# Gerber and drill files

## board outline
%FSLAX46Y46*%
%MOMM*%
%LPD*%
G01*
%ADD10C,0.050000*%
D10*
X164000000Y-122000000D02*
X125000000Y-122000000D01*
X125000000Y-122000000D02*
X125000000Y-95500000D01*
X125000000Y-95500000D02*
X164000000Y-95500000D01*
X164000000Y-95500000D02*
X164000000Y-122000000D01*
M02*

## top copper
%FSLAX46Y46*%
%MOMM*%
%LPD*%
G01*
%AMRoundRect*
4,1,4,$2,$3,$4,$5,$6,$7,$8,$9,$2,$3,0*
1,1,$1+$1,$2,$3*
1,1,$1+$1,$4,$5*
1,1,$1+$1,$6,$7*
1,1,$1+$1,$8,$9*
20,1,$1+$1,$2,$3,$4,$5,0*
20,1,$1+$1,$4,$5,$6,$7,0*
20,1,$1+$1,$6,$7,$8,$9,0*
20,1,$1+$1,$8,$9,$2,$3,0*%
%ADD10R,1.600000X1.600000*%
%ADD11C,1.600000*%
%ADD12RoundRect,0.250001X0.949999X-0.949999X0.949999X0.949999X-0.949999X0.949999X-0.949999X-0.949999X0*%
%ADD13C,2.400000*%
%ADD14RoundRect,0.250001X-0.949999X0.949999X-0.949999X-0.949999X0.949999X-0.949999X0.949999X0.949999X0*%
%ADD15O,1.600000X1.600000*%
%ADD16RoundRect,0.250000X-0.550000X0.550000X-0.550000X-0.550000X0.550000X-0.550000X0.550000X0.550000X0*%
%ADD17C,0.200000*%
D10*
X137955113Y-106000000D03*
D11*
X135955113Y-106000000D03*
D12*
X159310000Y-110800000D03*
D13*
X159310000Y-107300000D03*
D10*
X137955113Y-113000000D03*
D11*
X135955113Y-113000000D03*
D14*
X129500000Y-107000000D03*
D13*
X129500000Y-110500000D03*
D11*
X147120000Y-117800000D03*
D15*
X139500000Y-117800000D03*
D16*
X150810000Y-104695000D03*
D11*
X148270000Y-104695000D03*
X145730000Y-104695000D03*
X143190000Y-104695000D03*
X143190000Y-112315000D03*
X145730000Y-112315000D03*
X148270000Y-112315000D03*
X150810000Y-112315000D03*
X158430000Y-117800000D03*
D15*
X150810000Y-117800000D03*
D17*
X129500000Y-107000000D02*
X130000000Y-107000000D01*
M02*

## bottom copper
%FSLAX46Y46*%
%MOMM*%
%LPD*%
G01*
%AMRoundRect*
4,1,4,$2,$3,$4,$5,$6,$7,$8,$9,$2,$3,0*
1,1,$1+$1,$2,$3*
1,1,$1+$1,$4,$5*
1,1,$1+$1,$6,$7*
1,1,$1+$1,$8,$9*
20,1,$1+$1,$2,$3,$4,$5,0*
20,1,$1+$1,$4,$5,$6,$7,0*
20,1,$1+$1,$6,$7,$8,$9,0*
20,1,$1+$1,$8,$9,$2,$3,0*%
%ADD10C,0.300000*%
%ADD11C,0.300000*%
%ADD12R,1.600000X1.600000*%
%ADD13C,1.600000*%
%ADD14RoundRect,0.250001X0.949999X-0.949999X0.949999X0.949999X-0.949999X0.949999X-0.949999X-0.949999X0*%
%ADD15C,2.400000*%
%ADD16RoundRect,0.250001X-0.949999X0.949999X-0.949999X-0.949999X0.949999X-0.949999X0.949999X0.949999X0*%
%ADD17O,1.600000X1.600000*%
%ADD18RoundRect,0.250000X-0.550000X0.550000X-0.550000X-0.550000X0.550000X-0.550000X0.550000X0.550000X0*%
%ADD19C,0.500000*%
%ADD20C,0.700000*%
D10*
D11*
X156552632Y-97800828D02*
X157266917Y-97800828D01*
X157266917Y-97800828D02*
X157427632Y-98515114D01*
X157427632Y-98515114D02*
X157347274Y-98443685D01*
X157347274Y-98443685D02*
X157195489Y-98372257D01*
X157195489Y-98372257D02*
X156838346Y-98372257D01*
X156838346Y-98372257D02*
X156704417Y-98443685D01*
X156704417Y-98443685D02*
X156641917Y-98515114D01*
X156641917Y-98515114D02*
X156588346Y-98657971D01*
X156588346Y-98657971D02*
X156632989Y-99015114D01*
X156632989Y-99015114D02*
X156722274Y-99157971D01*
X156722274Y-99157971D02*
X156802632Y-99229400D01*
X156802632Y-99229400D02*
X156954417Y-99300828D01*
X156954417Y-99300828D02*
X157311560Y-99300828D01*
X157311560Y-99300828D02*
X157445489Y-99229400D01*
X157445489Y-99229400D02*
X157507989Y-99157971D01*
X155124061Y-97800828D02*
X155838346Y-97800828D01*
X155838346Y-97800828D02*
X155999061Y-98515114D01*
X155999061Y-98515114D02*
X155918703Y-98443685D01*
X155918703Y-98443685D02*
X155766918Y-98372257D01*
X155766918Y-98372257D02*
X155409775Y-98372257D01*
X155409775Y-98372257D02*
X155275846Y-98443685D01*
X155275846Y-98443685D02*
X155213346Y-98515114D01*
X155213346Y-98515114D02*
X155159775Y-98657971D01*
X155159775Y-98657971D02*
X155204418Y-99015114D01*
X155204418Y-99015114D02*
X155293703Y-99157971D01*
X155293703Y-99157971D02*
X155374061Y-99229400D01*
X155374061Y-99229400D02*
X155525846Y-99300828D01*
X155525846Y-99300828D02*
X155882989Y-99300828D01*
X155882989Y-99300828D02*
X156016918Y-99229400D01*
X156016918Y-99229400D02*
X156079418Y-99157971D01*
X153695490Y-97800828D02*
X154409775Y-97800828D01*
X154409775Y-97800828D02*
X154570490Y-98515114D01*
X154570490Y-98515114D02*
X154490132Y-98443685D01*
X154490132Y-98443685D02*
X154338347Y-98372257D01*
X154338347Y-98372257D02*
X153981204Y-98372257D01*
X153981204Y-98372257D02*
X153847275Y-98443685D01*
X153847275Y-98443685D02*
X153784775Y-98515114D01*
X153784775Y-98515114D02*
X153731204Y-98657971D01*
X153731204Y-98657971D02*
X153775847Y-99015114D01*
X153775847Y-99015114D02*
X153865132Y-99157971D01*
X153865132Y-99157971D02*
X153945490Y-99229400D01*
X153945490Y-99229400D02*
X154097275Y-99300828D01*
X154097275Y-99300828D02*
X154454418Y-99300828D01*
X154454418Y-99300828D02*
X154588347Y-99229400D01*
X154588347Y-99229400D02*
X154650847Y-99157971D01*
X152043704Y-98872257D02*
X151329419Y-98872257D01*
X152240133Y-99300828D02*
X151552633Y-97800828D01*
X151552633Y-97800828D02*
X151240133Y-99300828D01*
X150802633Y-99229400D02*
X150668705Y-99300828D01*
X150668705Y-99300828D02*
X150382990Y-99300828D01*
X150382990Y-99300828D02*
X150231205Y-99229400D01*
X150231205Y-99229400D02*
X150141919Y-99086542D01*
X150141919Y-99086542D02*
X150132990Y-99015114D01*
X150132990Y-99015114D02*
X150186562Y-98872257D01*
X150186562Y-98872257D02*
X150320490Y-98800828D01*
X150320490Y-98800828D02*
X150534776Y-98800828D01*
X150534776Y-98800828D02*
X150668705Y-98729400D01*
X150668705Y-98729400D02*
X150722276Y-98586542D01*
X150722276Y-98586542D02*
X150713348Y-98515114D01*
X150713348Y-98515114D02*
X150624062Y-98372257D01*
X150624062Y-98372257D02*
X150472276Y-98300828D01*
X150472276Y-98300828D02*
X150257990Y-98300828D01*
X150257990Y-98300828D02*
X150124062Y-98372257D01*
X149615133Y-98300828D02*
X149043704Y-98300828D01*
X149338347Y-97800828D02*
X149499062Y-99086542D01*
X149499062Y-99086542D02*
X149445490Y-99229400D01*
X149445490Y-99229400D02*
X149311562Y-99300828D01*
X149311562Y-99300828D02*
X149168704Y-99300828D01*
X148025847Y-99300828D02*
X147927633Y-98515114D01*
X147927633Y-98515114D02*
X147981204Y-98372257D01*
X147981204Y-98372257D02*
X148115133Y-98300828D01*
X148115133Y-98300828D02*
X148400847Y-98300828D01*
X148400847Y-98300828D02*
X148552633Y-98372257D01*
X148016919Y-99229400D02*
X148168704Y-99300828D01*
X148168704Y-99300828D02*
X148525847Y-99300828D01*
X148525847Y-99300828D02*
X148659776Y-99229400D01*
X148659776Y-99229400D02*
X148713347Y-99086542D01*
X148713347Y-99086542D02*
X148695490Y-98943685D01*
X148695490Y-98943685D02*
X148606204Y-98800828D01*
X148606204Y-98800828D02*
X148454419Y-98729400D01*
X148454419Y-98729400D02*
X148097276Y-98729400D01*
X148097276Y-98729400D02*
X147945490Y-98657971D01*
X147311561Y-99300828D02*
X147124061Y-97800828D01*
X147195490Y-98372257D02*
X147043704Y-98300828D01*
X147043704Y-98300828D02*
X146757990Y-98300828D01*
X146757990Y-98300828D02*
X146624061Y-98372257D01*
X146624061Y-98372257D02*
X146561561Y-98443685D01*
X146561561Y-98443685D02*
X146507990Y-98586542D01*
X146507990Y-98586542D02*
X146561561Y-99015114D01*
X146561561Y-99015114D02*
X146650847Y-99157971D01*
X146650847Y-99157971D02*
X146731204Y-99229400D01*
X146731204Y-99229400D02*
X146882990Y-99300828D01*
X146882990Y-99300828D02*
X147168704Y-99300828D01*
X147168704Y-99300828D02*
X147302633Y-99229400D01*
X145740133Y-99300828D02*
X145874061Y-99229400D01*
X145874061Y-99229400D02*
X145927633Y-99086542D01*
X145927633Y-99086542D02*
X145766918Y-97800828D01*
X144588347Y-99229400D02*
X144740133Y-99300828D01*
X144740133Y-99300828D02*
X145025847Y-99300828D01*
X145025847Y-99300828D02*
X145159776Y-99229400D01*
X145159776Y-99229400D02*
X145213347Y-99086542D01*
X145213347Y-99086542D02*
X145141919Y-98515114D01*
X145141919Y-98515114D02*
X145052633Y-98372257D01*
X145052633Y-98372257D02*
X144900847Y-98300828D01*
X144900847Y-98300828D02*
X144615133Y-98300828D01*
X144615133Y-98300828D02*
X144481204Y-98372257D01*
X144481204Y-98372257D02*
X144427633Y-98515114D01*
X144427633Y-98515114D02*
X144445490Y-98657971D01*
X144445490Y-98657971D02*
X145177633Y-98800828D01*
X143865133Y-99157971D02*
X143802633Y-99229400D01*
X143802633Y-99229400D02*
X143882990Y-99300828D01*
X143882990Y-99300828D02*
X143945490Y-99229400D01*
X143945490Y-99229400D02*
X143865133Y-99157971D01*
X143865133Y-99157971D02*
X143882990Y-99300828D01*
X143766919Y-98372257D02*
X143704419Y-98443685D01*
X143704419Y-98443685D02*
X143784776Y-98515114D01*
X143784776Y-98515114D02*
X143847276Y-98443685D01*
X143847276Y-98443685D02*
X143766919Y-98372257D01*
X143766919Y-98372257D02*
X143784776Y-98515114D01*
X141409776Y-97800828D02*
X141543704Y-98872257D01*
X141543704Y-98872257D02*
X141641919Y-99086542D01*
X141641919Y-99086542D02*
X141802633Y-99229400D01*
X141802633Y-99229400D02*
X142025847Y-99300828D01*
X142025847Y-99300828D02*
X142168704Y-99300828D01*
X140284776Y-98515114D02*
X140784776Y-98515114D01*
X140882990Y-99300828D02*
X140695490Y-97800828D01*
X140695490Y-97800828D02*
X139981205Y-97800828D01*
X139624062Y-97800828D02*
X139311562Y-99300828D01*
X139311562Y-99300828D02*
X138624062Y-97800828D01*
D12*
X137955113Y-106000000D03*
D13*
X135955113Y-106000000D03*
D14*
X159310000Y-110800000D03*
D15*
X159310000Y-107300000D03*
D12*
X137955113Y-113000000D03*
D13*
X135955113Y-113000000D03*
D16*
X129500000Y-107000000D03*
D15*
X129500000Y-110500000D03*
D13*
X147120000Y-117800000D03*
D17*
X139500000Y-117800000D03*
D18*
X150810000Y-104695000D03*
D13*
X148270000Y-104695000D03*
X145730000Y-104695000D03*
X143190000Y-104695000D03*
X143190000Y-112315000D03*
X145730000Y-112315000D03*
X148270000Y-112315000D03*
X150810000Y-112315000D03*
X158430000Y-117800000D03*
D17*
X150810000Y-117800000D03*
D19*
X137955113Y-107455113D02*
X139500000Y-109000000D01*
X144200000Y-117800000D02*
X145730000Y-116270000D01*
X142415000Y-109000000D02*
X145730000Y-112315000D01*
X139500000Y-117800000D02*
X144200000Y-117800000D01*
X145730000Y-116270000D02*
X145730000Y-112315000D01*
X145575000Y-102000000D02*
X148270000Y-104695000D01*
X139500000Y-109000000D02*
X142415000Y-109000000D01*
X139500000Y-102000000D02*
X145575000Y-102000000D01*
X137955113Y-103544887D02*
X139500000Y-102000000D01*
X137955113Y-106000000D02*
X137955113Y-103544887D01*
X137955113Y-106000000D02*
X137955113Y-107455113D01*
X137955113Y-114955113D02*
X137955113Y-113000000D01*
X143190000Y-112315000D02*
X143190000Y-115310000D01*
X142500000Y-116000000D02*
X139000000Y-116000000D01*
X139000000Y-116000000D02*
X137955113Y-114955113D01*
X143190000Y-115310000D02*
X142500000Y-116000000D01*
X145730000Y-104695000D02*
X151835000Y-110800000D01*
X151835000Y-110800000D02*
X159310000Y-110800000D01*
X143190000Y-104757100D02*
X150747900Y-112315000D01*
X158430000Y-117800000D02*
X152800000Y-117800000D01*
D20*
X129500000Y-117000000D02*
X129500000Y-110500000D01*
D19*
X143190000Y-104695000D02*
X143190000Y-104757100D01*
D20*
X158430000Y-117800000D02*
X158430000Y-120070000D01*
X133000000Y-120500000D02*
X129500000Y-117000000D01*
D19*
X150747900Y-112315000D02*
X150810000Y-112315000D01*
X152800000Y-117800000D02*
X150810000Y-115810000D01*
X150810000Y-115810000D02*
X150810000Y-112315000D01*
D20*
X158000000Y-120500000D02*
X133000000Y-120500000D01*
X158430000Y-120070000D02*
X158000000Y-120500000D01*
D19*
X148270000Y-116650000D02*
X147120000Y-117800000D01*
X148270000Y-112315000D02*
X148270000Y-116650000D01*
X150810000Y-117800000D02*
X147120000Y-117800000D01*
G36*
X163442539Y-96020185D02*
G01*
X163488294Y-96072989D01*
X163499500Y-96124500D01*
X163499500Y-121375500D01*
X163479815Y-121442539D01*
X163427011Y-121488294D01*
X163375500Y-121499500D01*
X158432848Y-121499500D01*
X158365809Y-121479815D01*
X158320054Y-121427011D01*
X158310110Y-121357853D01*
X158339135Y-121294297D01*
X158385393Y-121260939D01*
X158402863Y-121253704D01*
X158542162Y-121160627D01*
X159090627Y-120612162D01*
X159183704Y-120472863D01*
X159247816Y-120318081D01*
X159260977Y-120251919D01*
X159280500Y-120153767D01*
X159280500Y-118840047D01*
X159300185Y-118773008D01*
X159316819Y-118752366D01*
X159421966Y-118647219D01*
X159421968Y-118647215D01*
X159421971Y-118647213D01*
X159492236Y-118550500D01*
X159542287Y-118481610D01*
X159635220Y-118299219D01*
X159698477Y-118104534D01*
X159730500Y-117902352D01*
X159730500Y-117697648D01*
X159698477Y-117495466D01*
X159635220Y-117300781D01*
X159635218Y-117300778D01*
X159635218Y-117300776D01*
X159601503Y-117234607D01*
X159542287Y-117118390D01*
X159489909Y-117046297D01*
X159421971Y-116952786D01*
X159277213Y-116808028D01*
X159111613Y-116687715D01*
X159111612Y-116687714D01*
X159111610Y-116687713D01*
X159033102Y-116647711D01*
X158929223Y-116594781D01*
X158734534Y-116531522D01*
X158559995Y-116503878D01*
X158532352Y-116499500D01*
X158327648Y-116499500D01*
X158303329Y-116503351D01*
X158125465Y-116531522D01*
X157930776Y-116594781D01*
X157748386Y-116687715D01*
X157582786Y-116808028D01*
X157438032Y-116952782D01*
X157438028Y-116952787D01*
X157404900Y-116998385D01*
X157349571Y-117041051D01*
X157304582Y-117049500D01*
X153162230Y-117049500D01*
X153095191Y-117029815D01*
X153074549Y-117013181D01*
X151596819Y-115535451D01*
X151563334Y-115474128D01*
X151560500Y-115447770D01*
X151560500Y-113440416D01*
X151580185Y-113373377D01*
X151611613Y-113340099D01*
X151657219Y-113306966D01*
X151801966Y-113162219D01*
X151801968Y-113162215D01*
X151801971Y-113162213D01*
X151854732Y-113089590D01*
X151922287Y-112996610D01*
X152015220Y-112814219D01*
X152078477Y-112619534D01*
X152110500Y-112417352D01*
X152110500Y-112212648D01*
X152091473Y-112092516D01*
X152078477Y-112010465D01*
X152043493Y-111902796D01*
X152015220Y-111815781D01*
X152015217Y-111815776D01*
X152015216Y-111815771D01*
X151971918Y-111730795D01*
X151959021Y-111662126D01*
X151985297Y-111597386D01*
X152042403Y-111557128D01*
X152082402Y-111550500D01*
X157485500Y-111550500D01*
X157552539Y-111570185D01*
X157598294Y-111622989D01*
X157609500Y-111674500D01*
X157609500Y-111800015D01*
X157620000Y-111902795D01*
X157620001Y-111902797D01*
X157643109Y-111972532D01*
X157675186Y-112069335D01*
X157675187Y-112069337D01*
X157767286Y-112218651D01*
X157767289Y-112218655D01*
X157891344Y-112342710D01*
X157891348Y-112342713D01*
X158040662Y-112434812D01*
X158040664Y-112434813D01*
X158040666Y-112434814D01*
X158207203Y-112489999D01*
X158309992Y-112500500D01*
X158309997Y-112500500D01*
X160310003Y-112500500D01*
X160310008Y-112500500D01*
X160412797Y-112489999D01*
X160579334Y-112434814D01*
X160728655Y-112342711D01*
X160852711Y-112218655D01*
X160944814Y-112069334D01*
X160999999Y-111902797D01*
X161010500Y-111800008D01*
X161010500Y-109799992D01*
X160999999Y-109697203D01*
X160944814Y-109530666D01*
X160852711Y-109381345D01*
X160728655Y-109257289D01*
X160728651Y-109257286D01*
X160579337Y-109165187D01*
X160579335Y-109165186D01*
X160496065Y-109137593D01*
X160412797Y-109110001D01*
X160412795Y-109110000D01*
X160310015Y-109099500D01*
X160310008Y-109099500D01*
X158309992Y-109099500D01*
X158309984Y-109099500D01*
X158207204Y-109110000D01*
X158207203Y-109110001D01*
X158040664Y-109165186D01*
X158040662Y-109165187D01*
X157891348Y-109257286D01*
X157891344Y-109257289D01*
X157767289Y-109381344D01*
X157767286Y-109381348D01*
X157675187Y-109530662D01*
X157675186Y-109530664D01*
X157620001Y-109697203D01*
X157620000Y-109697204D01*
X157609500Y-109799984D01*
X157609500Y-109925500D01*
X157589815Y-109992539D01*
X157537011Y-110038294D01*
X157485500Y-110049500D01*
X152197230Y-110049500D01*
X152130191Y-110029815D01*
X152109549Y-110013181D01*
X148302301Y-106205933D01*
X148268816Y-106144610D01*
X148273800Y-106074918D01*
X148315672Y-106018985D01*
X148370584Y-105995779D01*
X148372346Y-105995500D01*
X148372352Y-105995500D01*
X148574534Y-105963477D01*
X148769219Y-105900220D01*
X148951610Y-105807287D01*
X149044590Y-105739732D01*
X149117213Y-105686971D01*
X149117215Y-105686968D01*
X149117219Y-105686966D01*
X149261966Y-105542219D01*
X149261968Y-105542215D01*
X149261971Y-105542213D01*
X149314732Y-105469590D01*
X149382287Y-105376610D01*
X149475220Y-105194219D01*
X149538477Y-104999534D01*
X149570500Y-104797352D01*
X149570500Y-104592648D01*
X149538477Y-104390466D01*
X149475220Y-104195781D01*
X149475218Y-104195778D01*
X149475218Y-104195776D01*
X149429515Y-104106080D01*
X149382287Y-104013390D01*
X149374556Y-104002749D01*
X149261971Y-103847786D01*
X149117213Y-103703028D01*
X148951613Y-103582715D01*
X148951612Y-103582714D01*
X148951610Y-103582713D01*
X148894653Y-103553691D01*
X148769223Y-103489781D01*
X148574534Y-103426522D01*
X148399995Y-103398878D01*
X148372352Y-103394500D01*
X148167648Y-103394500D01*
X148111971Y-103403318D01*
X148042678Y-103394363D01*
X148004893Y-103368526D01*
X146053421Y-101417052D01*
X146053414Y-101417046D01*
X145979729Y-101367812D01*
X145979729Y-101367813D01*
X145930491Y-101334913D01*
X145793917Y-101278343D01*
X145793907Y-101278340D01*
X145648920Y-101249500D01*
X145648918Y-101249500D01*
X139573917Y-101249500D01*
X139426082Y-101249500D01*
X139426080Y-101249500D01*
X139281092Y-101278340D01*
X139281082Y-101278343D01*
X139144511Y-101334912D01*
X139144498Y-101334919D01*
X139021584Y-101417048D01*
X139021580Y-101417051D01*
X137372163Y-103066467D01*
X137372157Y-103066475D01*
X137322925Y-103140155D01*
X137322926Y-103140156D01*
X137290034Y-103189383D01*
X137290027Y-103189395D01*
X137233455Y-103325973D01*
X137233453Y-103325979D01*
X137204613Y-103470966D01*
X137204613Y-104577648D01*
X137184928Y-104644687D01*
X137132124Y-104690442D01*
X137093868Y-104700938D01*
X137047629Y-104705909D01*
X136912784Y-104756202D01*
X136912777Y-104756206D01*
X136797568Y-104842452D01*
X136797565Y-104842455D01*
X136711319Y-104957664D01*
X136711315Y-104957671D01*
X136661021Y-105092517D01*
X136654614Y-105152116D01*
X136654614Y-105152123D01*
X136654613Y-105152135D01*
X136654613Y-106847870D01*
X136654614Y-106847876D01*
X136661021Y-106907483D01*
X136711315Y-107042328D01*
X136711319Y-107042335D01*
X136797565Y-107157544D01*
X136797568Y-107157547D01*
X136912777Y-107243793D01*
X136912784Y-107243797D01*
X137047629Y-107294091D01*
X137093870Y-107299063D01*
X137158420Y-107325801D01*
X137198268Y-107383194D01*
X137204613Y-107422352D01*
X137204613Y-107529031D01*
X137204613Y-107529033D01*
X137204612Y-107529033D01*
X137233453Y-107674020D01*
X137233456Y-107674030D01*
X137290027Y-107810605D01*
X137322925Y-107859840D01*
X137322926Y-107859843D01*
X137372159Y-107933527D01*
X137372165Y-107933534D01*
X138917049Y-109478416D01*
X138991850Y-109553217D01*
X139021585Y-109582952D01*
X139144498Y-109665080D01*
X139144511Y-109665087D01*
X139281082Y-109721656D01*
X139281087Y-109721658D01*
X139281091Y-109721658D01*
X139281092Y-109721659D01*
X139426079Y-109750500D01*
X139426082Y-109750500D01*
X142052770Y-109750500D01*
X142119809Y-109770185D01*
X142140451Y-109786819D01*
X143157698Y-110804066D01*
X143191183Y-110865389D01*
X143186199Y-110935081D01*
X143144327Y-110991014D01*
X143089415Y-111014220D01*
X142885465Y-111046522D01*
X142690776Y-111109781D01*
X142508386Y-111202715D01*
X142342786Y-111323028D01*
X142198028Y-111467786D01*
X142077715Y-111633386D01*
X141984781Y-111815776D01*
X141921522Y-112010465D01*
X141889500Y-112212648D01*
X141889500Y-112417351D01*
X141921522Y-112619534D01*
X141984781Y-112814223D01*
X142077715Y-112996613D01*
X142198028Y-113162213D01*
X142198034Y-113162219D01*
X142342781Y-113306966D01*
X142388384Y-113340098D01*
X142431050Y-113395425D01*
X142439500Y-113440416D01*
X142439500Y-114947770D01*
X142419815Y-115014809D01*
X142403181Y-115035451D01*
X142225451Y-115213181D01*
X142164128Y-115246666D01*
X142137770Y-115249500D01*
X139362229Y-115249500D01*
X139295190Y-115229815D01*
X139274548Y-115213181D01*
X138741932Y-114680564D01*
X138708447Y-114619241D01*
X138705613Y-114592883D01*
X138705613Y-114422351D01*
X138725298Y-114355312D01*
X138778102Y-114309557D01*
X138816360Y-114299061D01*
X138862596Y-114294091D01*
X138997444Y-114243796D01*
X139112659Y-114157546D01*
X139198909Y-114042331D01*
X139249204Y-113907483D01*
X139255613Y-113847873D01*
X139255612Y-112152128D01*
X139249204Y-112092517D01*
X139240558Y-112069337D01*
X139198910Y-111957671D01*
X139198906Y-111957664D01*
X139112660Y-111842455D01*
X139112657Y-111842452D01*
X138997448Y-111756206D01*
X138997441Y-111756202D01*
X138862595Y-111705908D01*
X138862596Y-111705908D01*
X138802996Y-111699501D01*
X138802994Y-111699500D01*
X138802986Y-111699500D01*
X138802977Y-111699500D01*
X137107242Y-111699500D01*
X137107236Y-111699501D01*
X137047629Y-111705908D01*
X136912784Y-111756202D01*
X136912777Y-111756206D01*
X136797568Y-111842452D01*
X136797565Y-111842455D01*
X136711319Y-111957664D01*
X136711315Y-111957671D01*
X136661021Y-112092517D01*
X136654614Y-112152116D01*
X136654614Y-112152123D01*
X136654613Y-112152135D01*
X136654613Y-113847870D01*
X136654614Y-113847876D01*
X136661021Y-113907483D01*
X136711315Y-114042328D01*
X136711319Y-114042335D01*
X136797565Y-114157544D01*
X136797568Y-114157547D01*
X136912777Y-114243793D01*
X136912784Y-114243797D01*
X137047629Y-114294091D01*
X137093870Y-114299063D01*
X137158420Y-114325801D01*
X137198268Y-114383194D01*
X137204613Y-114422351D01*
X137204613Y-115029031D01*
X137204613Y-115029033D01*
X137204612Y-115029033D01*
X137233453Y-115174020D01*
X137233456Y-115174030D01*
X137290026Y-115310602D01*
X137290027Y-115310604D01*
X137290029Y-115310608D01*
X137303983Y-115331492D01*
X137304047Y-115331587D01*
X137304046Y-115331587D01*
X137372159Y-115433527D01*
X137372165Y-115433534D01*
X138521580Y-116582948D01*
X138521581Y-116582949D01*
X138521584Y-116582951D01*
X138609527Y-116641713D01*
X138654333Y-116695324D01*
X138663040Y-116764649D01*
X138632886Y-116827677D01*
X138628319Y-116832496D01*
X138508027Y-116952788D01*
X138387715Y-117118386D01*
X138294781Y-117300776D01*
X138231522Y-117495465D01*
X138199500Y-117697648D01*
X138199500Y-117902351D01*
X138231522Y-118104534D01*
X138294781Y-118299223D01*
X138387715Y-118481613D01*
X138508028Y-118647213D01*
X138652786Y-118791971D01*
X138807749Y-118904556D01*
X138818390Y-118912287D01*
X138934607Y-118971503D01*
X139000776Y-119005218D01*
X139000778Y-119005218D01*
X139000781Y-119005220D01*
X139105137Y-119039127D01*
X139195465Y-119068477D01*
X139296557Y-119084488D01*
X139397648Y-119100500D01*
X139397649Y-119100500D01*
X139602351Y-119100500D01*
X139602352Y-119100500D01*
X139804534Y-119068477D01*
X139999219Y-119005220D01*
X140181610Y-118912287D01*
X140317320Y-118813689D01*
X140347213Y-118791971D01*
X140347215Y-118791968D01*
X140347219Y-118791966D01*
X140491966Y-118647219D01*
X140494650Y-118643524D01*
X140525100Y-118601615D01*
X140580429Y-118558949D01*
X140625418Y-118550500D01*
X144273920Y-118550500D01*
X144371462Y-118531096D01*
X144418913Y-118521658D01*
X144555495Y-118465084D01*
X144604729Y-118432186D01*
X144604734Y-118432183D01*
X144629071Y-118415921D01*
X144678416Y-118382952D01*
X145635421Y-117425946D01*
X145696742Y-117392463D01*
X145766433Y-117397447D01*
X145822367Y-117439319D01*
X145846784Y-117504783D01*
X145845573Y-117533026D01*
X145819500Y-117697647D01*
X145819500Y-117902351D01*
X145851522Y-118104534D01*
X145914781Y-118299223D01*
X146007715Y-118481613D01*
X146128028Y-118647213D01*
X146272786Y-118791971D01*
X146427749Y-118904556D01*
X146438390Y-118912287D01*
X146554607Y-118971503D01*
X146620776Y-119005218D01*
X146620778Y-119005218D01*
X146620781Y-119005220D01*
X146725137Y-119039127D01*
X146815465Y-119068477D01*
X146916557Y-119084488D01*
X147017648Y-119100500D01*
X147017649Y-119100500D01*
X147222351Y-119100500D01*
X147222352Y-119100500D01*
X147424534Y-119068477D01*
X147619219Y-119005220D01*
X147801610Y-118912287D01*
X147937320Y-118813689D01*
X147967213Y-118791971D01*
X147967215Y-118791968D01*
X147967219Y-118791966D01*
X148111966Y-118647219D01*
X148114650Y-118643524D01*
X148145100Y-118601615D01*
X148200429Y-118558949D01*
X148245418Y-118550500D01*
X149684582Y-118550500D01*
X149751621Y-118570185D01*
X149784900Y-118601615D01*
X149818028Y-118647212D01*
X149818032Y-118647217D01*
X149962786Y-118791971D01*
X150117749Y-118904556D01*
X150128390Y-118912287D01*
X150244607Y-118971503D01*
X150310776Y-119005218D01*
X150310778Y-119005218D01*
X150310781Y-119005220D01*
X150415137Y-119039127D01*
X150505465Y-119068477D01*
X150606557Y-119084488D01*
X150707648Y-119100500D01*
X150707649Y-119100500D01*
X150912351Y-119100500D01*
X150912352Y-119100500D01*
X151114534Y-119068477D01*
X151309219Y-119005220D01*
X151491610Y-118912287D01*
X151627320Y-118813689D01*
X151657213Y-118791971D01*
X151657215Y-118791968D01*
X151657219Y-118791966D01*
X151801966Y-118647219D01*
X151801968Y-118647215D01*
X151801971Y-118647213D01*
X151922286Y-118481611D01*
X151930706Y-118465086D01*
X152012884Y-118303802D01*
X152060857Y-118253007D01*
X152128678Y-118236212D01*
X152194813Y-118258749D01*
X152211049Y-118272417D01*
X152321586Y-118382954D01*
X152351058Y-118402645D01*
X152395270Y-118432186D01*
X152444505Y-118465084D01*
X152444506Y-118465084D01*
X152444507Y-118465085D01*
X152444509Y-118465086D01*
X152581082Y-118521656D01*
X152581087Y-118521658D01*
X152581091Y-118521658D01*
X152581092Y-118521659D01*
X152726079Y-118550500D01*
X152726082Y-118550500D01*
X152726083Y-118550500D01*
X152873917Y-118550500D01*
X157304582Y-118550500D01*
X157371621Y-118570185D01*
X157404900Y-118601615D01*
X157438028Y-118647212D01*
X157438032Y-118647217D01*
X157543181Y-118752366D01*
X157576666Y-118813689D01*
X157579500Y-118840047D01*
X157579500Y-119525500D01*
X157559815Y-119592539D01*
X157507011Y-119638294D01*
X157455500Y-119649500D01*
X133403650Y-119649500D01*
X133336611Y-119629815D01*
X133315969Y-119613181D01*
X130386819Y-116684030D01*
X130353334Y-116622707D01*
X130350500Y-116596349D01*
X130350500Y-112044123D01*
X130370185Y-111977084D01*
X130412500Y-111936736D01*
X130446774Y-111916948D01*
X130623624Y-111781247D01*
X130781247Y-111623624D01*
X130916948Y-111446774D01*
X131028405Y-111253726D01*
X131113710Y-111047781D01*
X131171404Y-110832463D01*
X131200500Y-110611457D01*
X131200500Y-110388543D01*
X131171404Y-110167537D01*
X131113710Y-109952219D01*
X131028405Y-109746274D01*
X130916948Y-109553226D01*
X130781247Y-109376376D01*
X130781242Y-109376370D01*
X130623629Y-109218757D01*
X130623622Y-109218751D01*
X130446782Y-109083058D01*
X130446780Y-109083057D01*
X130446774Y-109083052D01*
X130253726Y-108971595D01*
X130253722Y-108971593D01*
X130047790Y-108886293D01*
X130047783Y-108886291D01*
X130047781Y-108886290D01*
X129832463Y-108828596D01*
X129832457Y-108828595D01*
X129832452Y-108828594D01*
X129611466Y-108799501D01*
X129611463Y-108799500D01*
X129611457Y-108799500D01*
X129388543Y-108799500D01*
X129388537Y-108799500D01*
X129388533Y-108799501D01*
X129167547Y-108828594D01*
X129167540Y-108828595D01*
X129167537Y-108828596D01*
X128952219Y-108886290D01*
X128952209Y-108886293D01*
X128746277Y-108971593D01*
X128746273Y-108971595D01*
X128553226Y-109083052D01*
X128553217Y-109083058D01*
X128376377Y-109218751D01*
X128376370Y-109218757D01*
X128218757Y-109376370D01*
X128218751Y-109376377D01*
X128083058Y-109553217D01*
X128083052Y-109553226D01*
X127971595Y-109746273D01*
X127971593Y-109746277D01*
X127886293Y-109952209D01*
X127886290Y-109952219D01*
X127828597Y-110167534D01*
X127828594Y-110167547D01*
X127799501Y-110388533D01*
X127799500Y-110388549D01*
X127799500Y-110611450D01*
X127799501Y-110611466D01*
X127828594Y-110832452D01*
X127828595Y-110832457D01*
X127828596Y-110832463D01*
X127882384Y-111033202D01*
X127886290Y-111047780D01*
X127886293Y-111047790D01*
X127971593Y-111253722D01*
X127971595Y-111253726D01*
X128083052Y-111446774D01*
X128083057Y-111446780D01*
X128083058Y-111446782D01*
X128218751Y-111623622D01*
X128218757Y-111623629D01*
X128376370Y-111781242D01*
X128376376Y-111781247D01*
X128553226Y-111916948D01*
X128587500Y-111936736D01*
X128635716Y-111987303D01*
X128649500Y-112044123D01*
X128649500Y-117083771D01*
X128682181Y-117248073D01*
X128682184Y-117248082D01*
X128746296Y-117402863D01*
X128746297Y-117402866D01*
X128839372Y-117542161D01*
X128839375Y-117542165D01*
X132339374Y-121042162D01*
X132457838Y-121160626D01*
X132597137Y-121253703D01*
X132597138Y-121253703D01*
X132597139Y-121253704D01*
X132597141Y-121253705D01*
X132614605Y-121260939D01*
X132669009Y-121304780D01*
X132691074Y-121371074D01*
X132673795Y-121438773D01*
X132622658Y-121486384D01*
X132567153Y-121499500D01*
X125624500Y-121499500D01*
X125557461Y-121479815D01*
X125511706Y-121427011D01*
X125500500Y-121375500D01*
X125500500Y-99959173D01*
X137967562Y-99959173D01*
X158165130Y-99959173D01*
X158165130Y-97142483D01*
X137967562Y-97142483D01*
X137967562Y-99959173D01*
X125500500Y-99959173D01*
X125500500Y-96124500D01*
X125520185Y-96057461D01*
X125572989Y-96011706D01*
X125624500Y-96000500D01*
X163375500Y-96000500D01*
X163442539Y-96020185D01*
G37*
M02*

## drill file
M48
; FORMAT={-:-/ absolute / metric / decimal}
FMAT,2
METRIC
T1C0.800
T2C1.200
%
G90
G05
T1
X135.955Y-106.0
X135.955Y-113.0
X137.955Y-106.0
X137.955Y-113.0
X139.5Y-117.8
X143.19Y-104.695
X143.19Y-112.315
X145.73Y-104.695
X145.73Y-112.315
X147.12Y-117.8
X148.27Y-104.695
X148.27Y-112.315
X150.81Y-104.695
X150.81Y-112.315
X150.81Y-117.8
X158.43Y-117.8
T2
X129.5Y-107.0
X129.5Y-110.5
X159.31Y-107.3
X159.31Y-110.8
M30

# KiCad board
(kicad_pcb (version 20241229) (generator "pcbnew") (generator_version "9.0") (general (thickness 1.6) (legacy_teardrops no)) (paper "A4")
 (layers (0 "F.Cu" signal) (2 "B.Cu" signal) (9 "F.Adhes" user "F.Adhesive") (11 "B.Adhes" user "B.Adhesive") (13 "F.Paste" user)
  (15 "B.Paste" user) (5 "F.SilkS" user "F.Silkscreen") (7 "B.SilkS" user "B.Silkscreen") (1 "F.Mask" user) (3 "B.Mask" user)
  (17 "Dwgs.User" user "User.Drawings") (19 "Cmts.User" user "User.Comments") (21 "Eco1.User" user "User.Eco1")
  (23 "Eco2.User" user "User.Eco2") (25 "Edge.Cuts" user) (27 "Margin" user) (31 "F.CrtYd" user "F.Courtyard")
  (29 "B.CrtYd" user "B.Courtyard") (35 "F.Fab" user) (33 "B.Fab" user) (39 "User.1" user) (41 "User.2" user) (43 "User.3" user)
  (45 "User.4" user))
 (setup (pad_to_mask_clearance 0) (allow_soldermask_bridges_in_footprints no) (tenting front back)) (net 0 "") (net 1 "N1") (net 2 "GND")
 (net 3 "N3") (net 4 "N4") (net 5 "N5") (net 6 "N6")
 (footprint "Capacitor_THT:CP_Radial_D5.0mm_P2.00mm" (layer "F.Cu") (at 137.955113 106 180)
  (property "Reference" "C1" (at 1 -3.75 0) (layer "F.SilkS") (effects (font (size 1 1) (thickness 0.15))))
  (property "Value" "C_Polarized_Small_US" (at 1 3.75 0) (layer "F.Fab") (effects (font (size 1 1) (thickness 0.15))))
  (pad "1" thru_hole rect (at 0 0 180) (size 1.6 1.6) (drill 0.8) (layers "*.Cu" "*.Mask") (remove_unused_layers no) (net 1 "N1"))
  (pad "2" thru_hole circle (at 2 0 180) (size 1.6 1.6) (drill 0.8) (layers "*.Cu" "*.Mask") (remove_unused_layers no) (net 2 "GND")))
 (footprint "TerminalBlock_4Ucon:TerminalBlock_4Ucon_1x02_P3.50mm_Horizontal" (layer "F.Cu") (at 159.31 110.8 90)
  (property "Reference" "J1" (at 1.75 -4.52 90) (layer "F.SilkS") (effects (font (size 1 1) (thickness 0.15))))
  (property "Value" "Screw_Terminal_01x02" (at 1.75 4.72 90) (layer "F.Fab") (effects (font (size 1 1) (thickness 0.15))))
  (pad "1" thru_hole roundrect (at 0 0 90) (size 2.4 2.4) (drill 1.2) (layers "*.Cu" "*.Mask") (remove_unused_layers no)
   (roundrect_rratio 0.104167) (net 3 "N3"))
  (pad "2" thru_hole circle (at 3.5 0 90) (size 2.4 2.4) (drill 1.2) (layers "*.Cu" "*.Mask") (remove_unused_layers no) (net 2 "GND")))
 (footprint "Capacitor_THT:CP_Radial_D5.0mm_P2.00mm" (layer "F.Cu") (at 137.955113 113 180)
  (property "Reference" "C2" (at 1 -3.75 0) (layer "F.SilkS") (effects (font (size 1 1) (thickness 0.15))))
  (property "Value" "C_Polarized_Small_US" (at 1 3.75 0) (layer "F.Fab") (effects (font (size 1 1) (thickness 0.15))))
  (pad "1" thru_hole rect (at 0 0 180) (size 1.6 1.6) (drill 0.8) (layers "*.Cu" "*.Mask") (remove_unused_layers no) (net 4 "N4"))
  (pad "2" thru_hole circle (at 2 0 180) (size 1.6 1.6) (drill 0.8) (layers "*.Cu" "*.Mask") (remove_unused_layers no) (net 2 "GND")))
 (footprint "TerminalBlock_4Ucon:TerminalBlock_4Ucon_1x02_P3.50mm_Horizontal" (layer "F.Cu") (at 129.5 107 -90)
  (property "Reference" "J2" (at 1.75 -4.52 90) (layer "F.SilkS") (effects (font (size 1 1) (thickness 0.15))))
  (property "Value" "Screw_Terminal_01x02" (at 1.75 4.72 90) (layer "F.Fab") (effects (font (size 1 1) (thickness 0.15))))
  (pad "1" thru_hole roundrect (at 0 0 270) (size 2.4 2.4) (drill 1.2) (layers "*.Cu" "*.Mask") (remove_unused_layers no)
   (roundrect_rratio 0.104167) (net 2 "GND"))
  (pad "2" thru_hole circle (at 3.5 0 270) (size 2.4 2.4) (drill 1.2) (layers "*.Cu" "*.Mask") (remove_unused_layers no) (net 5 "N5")))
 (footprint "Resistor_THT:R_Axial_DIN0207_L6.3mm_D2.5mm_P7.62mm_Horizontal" (layer "F.Cu") (at 147.12 117.8 180)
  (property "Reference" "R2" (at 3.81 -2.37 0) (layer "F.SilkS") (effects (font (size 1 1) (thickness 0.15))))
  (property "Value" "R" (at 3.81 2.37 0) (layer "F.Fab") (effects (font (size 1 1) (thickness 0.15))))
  (pad "1" thru_hole circle (at 0 0 180) (size 1.6 1.6) (drill 0.8) (layers "*.Cu" "*.Mask") (remove_unused_layers no) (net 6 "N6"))
  (pad "2" thru_hole oval (at 7.62 0 180) (size 1.6 1.6) (drill 0.8) (layers "*.Cu" "*.Mask") (remove_unused_layers no) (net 1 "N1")))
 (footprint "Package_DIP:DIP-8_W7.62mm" (layer "F.Cu") (at 150.81 104.695 -90)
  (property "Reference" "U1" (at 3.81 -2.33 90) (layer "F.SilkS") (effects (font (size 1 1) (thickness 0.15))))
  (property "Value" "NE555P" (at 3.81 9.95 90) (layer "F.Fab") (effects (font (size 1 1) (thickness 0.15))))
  (pad "1" thru_hole roundrect (at 0 0 270) (size 1.6 1.6) (drill 0.8) (layers "*.Cu" "*.Mask") (remove_unused_layers no)
   (roundrect_rratio 0.15625) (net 2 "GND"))
  (pad "2" thru_hole circle (at 0 2.54 270) (size 1.6 1.6) (drill 0.8) (layers "*.Cu" "*.Mask") (remove_unused_layers no) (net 1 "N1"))
  (pad "3" thru_hole circle (at 0 5.08 270) (size 1.6 1.6) (drill 0.8) (layers "*.Cu" "*.Mask") (remove_unused_layers no) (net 3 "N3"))
  (pad "4" thru_hole circle (at 0 7.62 270) (size 1.6 1.6) (drill 0.8) (layers "*.Cu" "*.Mask") (remove_unused_layers no) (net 5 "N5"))
  (pad "5" thru_hole circle (at 7.62 7.62 270) (size 1.6 1.6) (drill 0.8) (layers "*.Cu" "*.Mask") (remove_unused_layers no) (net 4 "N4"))
  (pad "6" thru_hole circle (at 7.62 5.08 270) (size 1.6 1.6) (drill 0.8) (layers "*.Cu" "*.Mask") (remove_unused_layers no) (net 1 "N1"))
  (pad "7" thru_hole circle (at 7.62 2.54 270) (size 1.6 1.6) (drill 0.8) (layers "*.Cu" "*.Mask") (remove_unused_layers no) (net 6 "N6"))
  (pad "8" thru_hole circle (at 7.62 0 270) (size 1.6 1.6) (drill 0.8) (layers "*.Cu" "*.Mask") (remove_unused_layers no) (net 5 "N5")))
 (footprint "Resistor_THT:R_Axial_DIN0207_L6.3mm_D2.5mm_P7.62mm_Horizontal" (layer "F.Cu") (at 158.43 117.8 180)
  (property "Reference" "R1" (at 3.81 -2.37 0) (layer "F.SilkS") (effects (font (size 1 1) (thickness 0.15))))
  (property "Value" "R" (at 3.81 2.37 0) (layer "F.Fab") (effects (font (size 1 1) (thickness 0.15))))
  (pad "1" thru_hole circle (at 0 0 180) (size 1.6 1.6) (drill 0.8) (layers "*.Cu" "*.Mask") (remove_unused_layers no) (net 5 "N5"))
  (pad "2" thru_hole oval (at 7.62 0 180) (size 1.6 1.6) (drill 0.8) (layers "*.Cu" "*.Mask") (remove_unused_layers no) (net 6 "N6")))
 (gr_line (start 164 122) (end 125 122) (stroke (width 0.05) (type default)) (layer "Edge.Cuts"))
 (gr_line (start 125 122) (end 125 95.5) (stroke (width 0.05) (type default)) (layer "Edge.Cuts"))
 (gr_line (start 125 95.5) (end 164 95.5) (stroke (width 0.05) (type default)) (layer "Edge.Cuts"))
 (gr_line (start 164 95.5) (end 164 122) (stroke (width 0.05) (type default)) (layer "Edge.Cuts"))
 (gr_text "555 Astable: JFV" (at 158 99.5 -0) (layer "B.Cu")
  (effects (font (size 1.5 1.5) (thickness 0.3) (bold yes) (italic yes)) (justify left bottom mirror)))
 (segment (start 137.955113 107.455113) (end 139.5 109) (width 0.5) (layer "B.Cu") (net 1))
 (segment (start 144.2 117.8) (end 145.73 116.27) (width 0.5) (layer "B.Cu") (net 1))
 (segment (start 142.415 109) (end 145.73 112.315) (width 0.5) (layer "B.Cu") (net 1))
 (segment (start 139.5 117.8) (end 144.2 117.8) (width 0.5) (layer "B.Cu") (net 1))
 (segment (start 145.73 116.27) (end 145.73 112.315) (width 0.5) (layer "B.Cu") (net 1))
 (segment (start 145.575 102) (end 148.27 104.695) (width 0.5) (layer "B.Cu") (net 1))
 (segment (start 139.5 109) (end 142.415 109) (width 0.5) (layer "B.Cu") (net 1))
 (segment (start 139.5 102) (end 145.575 102) (width 0.5) (layer "B.Cu") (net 1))
 (segment (start 137.955113 103.544887) (end 139.5 102) (width 0.5) (layer "B.Cu") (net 1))
 (segment (start 137.955113 106) (end 137.955113 103.544887) (width 0.5) (layer "B.Cu") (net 1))
 (segment (start 137.955113 106) (end 137.955113 107.455113) (width 0.5) (layer "B.Cu") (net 1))
 (segment (start 129.5 107) (end 130 107) (width 0.2) (layer "F.Cu") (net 2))
 (segment (start 137.955113 114.955113) (end 137.955113 113) (width 0.5) (layer "B.Cu") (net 4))
 (segment (start 143.19 112.315) (end 143.19 115.31) (width 0.5) (layer "B.Cu") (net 4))
 (segment (start 142.5 116) (end 139 116) (width 0.5) (layer "B.Cu") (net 4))
 (segment (start 139 116) (end 137.955113 114.955113) (width 0.5) (layer "B.Cu") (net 4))
 (segment (start 143.19 115.31) (end 142.5 116) (width 0.5) (layer "B.Cu") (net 4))
 (segment (start 145.73 104.695) (end 151.835 110.8) (width 0.5) (layer "B.Cu") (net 3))
 (segment (start 151.835 110.8) (end 159.31 110.8) (width 0.5) (layer "B.Cu") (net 3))
 (segment (start 143.19 104.7571) (end 150.7479 112.315) (width 0.5) (layer "B.Cu") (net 5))
 (segment (start 158.43 117.8) (end 152.8 117.8) (width 0.5) (layer "B.Cu") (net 5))
 (segment (start 129.5 117) (end 129.5 110.5) (width 0.7) (layer "B.Cu") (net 5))
 (segment (start 143.19 104.695) (end 143.19 104.7571) (width 0.5) (layer "B.Cu") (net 5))
 (segment (start 158.43 117.8) (end 158.43 120.07) (width 0.7) (layer "B.Cu") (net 5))
 (segment (start 133 120.5) (end 129.5 117) (width 0.7) (layer "B.Cu") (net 5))
 (segment (start 150.7479 112.315) (end 150.81 112.315) (width 0.5) (layer "B.Cu") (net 5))
 (segment (start 152.8 117.8) (end 150.81 115.81) (width 0.5) (layer "B.Cu") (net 5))
 (segment (start 150.81 115.81) (end 150.81 112.315) (width 0.5) (layer "B.Cu") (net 5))
 (segment (start 158 120.5) (end 133 120.5) (width 0.7) (layer "B.Cu") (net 5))
 (segment (start 158.43 120.07) (end 158 120.5) (width 0.7) (layer "B.Cu") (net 5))
 (segment (start 148.27 116.65) (end 147.12 117.8) (width 0.5) (layer "B.Cu") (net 6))
 (segment (start 148.27 112.315) (end 148.27 116.65) (width 0.5) (layer "B.Cu") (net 6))
 (segment (start 150.81 117.8) (end 147.12 117.8) (width 0.5) (layer "B.Cu") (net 6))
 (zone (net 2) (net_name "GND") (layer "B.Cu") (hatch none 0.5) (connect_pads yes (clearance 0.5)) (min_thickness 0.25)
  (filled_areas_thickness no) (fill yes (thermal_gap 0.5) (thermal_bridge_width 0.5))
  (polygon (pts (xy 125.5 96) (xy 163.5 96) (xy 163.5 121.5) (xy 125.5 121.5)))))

